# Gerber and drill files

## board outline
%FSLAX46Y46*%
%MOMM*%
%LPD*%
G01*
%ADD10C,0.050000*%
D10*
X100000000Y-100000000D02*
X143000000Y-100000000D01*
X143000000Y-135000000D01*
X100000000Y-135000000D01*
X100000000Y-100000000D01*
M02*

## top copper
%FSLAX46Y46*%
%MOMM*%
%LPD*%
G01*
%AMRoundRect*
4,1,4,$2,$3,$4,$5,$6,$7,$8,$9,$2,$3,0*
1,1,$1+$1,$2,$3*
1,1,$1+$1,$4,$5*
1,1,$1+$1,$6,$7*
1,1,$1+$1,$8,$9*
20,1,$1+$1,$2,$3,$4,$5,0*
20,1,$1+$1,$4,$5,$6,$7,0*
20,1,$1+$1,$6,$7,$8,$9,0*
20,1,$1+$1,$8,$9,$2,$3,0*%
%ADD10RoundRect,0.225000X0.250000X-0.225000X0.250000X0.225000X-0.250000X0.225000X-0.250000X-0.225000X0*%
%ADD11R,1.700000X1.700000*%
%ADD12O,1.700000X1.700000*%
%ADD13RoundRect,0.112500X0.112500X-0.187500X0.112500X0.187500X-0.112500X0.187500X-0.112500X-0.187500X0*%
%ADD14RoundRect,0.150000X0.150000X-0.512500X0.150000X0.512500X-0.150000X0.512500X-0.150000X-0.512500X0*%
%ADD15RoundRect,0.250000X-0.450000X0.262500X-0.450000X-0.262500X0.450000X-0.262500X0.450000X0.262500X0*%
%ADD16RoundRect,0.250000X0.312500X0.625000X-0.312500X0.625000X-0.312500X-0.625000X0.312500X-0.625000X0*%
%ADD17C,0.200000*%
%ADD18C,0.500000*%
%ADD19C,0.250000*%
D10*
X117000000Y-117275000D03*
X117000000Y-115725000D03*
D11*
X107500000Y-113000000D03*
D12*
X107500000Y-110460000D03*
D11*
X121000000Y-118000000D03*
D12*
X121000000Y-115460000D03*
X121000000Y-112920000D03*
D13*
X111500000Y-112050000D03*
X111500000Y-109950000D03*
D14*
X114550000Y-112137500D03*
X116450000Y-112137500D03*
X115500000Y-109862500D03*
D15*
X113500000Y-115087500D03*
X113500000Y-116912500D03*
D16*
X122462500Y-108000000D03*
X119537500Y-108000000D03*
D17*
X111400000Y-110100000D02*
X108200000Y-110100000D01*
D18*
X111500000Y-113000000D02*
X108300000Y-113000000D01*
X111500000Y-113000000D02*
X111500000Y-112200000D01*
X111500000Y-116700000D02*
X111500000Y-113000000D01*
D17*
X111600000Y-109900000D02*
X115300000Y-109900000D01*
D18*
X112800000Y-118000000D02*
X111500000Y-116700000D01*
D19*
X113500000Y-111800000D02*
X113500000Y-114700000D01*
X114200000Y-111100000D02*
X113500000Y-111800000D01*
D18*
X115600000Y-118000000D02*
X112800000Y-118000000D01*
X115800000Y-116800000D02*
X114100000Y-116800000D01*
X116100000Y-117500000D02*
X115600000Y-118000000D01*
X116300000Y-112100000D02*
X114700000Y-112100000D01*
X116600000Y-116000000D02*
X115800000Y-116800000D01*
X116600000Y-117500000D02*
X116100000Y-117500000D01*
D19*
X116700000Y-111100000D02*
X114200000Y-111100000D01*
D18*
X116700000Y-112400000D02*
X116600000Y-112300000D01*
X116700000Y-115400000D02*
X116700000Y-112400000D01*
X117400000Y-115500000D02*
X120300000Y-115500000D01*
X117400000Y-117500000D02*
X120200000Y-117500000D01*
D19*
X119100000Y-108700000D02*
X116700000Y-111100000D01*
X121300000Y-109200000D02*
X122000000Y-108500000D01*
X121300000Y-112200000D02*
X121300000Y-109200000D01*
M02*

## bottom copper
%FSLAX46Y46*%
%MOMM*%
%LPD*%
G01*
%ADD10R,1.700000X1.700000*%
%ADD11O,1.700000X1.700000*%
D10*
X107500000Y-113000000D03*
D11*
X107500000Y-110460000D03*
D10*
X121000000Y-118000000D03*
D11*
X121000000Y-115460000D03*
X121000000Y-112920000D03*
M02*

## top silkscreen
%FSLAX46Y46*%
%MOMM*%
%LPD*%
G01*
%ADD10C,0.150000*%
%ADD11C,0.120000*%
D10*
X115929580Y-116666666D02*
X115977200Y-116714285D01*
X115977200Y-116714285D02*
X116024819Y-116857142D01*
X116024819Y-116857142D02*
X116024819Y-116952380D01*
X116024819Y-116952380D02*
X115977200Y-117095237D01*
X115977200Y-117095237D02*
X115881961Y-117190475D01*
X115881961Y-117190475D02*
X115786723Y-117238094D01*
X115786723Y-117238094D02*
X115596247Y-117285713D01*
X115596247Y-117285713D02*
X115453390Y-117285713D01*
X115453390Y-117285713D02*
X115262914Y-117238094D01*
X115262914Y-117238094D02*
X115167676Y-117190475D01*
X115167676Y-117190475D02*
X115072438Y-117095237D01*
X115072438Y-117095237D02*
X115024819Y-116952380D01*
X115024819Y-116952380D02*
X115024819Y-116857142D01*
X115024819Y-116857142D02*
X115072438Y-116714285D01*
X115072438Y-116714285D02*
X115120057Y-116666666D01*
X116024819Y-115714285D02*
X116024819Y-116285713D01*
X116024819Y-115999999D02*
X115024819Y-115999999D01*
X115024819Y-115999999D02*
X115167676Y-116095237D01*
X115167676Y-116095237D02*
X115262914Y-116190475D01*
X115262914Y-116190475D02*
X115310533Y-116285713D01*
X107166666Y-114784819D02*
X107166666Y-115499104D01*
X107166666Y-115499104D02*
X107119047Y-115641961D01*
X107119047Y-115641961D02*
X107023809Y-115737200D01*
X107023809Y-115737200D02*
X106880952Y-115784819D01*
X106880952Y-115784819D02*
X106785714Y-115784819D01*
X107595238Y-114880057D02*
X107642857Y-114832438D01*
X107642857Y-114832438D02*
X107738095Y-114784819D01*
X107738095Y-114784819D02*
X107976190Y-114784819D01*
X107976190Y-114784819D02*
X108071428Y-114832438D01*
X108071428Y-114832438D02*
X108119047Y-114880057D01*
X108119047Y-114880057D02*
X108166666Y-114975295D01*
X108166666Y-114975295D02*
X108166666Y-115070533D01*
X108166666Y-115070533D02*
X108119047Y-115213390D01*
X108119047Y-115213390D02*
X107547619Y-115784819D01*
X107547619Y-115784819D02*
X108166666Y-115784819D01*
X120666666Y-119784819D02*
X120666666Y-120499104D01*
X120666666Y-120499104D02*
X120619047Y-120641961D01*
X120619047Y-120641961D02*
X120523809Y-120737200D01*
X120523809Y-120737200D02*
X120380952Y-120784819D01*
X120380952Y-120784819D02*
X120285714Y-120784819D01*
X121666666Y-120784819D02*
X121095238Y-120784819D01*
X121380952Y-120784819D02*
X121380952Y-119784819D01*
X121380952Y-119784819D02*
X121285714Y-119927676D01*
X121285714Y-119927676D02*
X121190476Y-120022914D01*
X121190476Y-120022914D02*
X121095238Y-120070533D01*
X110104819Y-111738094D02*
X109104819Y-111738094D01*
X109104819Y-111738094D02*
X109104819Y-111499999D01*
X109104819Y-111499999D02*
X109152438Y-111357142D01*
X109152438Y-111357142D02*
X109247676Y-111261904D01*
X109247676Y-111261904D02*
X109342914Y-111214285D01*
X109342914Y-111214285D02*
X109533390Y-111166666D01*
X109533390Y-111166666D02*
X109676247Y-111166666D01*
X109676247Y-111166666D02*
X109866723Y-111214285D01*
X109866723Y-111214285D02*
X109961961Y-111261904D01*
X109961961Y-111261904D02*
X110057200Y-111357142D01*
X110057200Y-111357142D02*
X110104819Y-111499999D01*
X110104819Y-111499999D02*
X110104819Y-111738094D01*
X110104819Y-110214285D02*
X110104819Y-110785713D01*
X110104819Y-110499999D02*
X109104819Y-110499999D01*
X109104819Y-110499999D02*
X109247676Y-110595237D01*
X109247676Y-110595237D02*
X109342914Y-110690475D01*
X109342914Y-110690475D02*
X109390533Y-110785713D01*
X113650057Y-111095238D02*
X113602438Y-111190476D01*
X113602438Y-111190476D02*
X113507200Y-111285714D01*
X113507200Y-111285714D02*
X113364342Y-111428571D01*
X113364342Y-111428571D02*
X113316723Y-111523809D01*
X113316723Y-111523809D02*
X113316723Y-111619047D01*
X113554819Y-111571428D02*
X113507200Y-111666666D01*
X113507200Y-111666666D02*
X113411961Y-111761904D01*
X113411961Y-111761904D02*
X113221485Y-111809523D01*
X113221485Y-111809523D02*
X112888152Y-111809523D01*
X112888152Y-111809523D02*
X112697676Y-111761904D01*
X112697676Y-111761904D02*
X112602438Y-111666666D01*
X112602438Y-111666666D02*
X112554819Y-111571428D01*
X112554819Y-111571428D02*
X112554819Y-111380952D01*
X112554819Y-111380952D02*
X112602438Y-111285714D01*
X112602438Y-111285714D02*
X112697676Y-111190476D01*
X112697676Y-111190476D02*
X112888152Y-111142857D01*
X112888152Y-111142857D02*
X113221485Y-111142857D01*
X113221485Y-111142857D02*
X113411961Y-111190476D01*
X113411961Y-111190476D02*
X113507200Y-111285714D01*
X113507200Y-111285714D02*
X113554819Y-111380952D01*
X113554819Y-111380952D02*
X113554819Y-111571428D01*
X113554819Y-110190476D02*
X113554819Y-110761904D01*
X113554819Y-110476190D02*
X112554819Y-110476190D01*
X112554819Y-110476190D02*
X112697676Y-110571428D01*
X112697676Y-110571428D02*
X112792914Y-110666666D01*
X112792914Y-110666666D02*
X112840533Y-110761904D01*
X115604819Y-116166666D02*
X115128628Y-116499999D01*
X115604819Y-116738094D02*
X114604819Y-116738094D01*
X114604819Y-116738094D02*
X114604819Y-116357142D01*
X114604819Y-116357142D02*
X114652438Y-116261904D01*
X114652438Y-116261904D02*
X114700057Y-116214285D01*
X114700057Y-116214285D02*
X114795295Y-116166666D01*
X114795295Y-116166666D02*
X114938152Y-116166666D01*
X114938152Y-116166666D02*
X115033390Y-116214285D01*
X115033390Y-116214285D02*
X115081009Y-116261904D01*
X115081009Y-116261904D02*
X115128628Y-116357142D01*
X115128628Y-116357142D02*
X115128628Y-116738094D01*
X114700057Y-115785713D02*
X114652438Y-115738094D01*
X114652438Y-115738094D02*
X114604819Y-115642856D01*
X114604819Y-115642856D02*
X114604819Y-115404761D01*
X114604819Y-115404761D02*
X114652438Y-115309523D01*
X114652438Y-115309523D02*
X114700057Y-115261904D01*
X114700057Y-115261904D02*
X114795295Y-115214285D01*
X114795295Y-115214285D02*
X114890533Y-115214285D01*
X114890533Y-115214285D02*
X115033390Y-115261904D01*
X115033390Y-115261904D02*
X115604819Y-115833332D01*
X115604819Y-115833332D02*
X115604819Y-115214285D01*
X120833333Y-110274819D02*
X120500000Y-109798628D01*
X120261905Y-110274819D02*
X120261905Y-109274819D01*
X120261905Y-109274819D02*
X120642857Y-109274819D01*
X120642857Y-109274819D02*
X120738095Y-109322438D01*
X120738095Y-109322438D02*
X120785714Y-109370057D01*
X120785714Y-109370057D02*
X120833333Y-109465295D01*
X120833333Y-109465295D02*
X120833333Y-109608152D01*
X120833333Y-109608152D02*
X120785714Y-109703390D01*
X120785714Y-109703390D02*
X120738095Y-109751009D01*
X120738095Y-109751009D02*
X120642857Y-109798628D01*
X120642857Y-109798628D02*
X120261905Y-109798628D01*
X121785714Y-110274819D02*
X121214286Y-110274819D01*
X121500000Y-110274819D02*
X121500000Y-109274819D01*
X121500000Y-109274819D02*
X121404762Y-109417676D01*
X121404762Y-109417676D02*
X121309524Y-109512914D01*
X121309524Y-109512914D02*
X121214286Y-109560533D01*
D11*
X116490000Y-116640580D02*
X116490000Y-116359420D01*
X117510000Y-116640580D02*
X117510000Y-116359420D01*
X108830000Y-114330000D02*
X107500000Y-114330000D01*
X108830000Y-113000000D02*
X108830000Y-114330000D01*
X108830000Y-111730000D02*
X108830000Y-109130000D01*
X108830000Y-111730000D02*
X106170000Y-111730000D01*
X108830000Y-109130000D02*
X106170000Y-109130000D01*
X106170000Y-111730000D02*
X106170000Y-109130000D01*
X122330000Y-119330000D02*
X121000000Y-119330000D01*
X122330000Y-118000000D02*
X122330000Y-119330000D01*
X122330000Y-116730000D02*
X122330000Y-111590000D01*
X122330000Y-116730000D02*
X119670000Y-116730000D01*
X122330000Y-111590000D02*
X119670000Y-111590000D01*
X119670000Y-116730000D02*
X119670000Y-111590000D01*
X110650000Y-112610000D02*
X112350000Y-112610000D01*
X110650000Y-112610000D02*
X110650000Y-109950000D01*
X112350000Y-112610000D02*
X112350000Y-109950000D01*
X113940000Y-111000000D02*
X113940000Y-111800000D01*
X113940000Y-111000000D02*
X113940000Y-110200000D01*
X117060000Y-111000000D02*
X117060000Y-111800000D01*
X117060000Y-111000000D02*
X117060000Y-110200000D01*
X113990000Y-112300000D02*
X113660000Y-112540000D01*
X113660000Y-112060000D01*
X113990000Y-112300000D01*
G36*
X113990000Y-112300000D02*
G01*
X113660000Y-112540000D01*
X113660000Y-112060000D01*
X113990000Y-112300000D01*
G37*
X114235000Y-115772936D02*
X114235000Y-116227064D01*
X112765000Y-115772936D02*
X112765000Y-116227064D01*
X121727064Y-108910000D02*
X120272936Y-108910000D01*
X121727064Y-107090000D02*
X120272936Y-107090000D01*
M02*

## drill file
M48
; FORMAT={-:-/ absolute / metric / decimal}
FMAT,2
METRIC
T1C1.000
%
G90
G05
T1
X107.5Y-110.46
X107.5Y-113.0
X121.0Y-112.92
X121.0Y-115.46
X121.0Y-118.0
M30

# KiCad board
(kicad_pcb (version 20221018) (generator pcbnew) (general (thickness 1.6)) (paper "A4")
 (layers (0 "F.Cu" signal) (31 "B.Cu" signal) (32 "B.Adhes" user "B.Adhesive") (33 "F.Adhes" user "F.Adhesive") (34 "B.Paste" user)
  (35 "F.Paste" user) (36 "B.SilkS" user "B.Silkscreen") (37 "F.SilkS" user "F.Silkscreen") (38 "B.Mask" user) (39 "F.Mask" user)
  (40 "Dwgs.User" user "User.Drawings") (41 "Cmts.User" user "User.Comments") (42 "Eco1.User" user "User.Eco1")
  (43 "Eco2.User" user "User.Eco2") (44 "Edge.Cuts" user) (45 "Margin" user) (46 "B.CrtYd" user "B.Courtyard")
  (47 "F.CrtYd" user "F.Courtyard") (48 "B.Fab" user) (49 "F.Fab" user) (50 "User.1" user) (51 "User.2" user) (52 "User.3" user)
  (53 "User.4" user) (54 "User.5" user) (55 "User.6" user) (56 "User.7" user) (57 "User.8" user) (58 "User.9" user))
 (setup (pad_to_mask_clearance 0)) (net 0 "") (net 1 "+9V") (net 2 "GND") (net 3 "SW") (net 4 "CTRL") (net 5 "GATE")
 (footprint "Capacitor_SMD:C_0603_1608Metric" (layer "F.Cu") (at 117 116.5 90)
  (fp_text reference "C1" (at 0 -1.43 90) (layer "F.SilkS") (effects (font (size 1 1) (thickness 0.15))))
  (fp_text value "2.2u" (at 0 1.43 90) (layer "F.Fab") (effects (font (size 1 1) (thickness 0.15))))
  (fp_line (start -0.14058 -0.51) (end 0.14058 -0.51) (stroke (width 0.12) (type solid)) (layer "F.SilkS"))
  (fp_line (start -0.14058 0.51) (end 0.14058 0.51) (stroke (width 0.12) (type solid)) (layer "F.SilkS"))
  (pad "1" smd roundrect (at -0.775 0 90) (size 0.9 0.95) (layers "F.Cu" "F.Paste" "F.Mask") (roundrect_rratio 0.25) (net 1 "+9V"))
  (pad "2" smd roundrect (at 0.775 0 90) (size 0.9 0.95) (layers "F.Cu" "F.Paste" "F.Mask") (roundrect_rratio 0.25) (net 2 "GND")))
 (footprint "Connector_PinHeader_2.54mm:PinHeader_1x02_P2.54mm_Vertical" (layer "F.Cu") (at 107.5 113 180)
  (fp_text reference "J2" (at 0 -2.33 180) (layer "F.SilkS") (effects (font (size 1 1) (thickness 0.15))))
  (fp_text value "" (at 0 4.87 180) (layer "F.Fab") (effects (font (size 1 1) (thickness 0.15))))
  (fp_line (start -1.33 -1.33) (end 0 -1.33) (stroke (width 0.12) (type solid)) (layer "F.SilkS"))
  (fp_line (start -1.33 0) (end -1.33 -1.33) (stroke (width 0.12) (type solid)) (layer "F.SilkS"))
  (fp_line (start -1.33 1.27) (end -1.33 3.87) (stroke (width 0.12) (type solid)) (layer "F.SilkS"))
  (fp_line (start -1.33 1.27) (end 1.33 1.27) (stroke (width 0.12) (type solid)) (layer "F.SilkS"))
  (fp_line (start -1.33 3.87) (end 1.33 3.87) (stroke (width 0.12) (type solid)) (layer "F.SilkS"))
  (fp_line (start 1.33 1.27) (end 1.33 3.87) (stroke (width 0.12) (type solid)) (layer "F.SilkS"))
  (pad "1" thru_hole rect (at 0 0 180) (size 1.7 1.7) (drill 1) (layers "*.Cu" "*.Mask") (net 1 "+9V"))
  (pad "2" thru_hole oval (at 0 2.54 180) (size 1.7 1.7) (drill 1) (layers "*.Cu" "*.Mask") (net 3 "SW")))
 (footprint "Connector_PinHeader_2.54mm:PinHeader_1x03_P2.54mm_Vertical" (layer "F.Cu") (at 121 118 180)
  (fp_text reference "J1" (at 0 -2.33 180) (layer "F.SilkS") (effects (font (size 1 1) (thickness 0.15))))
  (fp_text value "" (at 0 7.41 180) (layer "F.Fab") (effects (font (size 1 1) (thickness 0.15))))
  (fp_line (start -1.33 -1.33) (end 0 -1.33) (stroke (width 0.12) (type solid)) (layer "F.SilkS"))
  (fp_line (start -1.33 0) (end -1.33 -1.33) (stroke (width 0.12) (type solid)) (layer "F.SilkS"))
  (fp_line (start -1.33 1.27) (end -1.33 6.41) (stroke (width 0.12) (type solid)) (layer "F.SilkS"))
  (fp_line (start -1.33 1.27) (end 1.33 1.27) (stroke (width 0.12) (type solid)) (layer "F.SilkS"))
  (fp_line (start -1.33 6.41) (end 1.33 6.41) (stroke (width 0.12) (type solid)) (layer "F.SilkS"))
  (fp_line (start 1.33 1.27) (end 1.33 6.41) (stroke (width 0.12) (type solid)) (layer "F.SilkS"))
  (pad "1" thru_hole rect (at 0 0 180) (size 1.7 1.7) (drill 1) (layers "*.Cu" "*.Mask") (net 1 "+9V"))
  (pad "2" thru_hole oval (at 0 2.54 180) (size 1.7 1.7) (drill 1) (layers "*.Cu" "*.Mask") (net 2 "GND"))
  (pad "3" thru_hole oval (at 0 5.08 180) (size 1.7 1.7) (drill 1) (layers "*.Cu" "*.Mask") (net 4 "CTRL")))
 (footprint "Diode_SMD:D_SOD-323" (layer "F.Cu") (at 111.5 111 90)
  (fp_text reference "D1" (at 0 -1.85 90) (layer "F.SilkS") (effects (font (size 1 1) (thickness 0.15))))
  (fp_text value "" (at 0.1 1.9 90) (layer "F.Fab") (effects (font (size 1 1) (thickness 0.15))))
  (fp_line (start -1.61 -0.85) (end -1.61 0.85) (stroke (width 0.12) (type solid)) (layer "F.SilkS"))
  (fp_line (start -1.61 -0.85) (end 1.05 -0.85) (stroke (width 0.12) (type solid)) (layer "F.SilkS"))
  (fp_line (start -1.61 0.85) (end 1.05 0.85) (stroke (width 0.12) (type solid)) (layer "F.SilkS"))
  (pad "1" smd roundrect (at -1.05 0 90) (size 0.6 0.45) (layers "F.Cu" "F.Paste" "F.Mask") (roundrect_rratio 0.25) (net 1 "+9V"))
  (pad "2" smd roundrect (at 1.05 0 90) (size 0.6 0.45) (layers "F.Cu" "F.Paste" "F.Mask") (roundrect_rratio 0.25) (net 3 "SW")))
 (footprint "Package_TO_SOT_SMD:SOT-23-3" (layer "F.Cu") (at 115.5 111 90)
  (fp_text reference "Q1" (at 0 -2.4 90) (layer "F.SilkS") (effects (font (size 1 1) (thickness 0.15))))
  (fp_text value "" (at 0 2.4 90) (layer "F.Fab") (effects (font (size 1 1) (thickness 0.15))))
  (fp_line (start 0 -1.56) (end -0.8 -1.56) (stroke (width 0.12) (type solid)) (layer "F.SilkS"))
  (fp_line (start 0 -1.56) (end 0.8 -1.56) (stroke (width 0.12) (type solid)) (layer "F.SilkS"))
  (fp_line (start 0 1.56) (end -0.8 1.56) (stroke (width 0.12) (type solid)) (layer "F.SilkS"))
  (fp_line (start 0 1.56) (end 0.8 1.56) (stroke (width 0.12) (type solid)) (layer "F.SilkS"))
  (fp_poly
   (pts (xy -1.3 -1.51) (xy -1.54 -1.84) (xy -1.06 -1.84) (xy -1.3 -1.51)) (stroke (width 0.12) (type solid)) (fill solid) (layer "F.SilkS"))
  (pad "1" smd roundrect (at -1.1375 -0.95 90) (size 1.325 0.6) (layers "F.Cu" "F.Paste" "F.Mask") (roundrect_rratio 0.25) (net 2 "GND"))
  (pad "2" smd roundrect (at -1.1375 0.95 90) (size 1.325 0.6) (layers "F.Cu" "F.Paste" "F.Mask") (roundrect_rratio 0.25) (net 2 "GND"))
  (pad "3" smd roundrect (at 1.1375 0 90) (size 1.325 0.6) (layers "F.Cu" "F.Paste" "F.Mask") (roundrect_rratio 0.25) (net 3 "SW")))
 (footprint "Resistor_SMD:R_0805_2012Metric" (layer "F.Cu") (at 113.5 116 -90)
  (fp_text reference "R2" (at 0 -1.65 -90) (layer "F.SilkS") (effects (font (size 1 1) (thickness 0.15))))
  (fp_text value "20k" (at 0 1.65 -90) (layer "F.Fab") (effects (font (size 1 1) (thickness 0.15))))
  (fp_line (start -0.227064 -0.735) (end 0.227064 -0.735) (stroke (width 0.12) (type solid)) (layer "F.SilkS"))
  (fp_line (start -0.227064 0.735) (end 0.227064 0.735) (stroke (width 0.12) (type solid)) (layer "F.SilkS"))
  (pad "1" smd roundrect (at -0.9125 0 270) (size 1.025 1.4) (layers "F.Cu" "F.Paste" "F.Mask") (roundrect_rratio 0.243902) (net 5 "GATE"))
  (pad "2" smd roundrect (at 0.9125 0 270) (size 1.025 1.4) (layers "F.Cu" "F.Paste" "F.Mask") (roundrect_rratio 0.243902) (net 2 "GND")))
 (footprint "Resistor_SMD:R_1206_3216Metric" (layer "F.Cu") (at 121 108 180)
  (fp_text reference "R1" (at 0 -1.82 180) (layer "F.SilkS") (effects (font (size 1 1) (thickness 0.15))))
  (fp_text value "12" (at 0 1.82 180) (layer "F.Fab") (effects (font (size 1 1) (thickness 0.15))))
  (fp_line (start -0.727064 -0.91) (end 0.727064 -0.91) (stroke (width 0.12) (type solid)) (layer "F.SilkS"))
  (fp_line (start -0.727064 0.91) (end 0.727064 0.91) (stroke (width 0.12) (type solid)) (layer "F.SilkS"))
  (pad "1" smd roundrect (at -1.4625 0 180) (size 1.125 1.75) (layers "F.Cu" "F.Paste" "F.Mask") (roundrect_rratio 0.222222) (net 4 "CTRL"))
  (pad "2" smd roundrect (at 1.4625 0 180) (size 1.125 1.75) (layers "F.Cu" "F.Paste" "F.Mask") (roundrect_rratio 0.222222) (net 5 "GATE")))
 (gr_rect (start 100 100) (end 143 135) (stroke (width 0.05) (type default)) (fill none) (layer "Edge.Cuts"))
 (segment (start 111.4 110.1) (end 108.2 110.1) (width 0.2) (layer "F.Cu") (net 3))
 (segment (start 111.5 113) (end 108.3 113) (width 0.5) (layer "F.Cu") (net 1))
 (segment (start 111.5 113) (end 111.5 112.2) (width 0.5) (layer "F.Cu") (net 1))
 (segment (start 111.5 116.7) (end 111.5 113) (width 0.5) (layer "F.Cu") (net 1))
 (segment (start 111.6 109.9) (end 115.3 109.9) (width 0.2) (layer "F.Cu") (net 3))
 (segment (start 112.8 118) (end 111.5 116.7) (width 0.5) (layer "F.Cu") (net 1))
 (segment (start 113.5 111.8) (end 113.5 114.7) (width 0.25) (layer "F.Cu") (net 5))
 (segment (start 114.2 111.1) (end 113.5 111.8) (width 0.25) (layer "F.Cu") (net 5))
 (segment (start 115.6 118) (end 112.8 118) (width 0.5) (layer "F.Cu") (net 1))
 (segment (start 115.8 116.8) (end 114.1 116.8) (width 0.5) (layer "F.Cu") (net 2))
 (segment (start 116.1 117.5) (end 115.6 118) (width 0.5) (layer "F.Cu") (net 1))
 (segment (start 116.3 112.1) (end 114.7 112.1) (width 0.5) (layer "F.Cu") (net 2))
 (segment (start 116.6 116) (end 115.8 116.8) (width 0.5) (layer "F.Cu") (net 2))
 (segment (start 116.6 117.5) (end 116.1 117.5) (width 0.5) (layer "F.Cu") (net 1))
 (segment (start 116.7 111.1) (end 114.2 111.1) (width 0.25) (layer "F.Cu") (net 5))
 (segment (start 116.7 112.4) (end 116.6 112.3) (width 0.5) (layer "F.Cu") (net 2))
 (segment (start 116.7 115.4) (end 116.7 112.4) (width 0.5) (layer "F.Cu") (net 2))
 (segment (start 117.4 115.5) (end 120.3 115.5) (width 0.5) (layer "F.Cu") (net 2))
 (segment (start 117.4 117.5) (end 120.2 117.5) (width 0.5) (layer "F.Cu") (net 1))
 (segment (start 119.1 108.7) (end 116.7 111.1) (width 0.25) (layer "F.Cu") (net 5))
 (segment (start 121.3 109.2) (end 122 108.5) (width 0.25) (layer "F.Cu") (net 4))
 (segment (start 121.3 112.2) (end 121.3 109.2) (width 0.25) (layer "F.Cu") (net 4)))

